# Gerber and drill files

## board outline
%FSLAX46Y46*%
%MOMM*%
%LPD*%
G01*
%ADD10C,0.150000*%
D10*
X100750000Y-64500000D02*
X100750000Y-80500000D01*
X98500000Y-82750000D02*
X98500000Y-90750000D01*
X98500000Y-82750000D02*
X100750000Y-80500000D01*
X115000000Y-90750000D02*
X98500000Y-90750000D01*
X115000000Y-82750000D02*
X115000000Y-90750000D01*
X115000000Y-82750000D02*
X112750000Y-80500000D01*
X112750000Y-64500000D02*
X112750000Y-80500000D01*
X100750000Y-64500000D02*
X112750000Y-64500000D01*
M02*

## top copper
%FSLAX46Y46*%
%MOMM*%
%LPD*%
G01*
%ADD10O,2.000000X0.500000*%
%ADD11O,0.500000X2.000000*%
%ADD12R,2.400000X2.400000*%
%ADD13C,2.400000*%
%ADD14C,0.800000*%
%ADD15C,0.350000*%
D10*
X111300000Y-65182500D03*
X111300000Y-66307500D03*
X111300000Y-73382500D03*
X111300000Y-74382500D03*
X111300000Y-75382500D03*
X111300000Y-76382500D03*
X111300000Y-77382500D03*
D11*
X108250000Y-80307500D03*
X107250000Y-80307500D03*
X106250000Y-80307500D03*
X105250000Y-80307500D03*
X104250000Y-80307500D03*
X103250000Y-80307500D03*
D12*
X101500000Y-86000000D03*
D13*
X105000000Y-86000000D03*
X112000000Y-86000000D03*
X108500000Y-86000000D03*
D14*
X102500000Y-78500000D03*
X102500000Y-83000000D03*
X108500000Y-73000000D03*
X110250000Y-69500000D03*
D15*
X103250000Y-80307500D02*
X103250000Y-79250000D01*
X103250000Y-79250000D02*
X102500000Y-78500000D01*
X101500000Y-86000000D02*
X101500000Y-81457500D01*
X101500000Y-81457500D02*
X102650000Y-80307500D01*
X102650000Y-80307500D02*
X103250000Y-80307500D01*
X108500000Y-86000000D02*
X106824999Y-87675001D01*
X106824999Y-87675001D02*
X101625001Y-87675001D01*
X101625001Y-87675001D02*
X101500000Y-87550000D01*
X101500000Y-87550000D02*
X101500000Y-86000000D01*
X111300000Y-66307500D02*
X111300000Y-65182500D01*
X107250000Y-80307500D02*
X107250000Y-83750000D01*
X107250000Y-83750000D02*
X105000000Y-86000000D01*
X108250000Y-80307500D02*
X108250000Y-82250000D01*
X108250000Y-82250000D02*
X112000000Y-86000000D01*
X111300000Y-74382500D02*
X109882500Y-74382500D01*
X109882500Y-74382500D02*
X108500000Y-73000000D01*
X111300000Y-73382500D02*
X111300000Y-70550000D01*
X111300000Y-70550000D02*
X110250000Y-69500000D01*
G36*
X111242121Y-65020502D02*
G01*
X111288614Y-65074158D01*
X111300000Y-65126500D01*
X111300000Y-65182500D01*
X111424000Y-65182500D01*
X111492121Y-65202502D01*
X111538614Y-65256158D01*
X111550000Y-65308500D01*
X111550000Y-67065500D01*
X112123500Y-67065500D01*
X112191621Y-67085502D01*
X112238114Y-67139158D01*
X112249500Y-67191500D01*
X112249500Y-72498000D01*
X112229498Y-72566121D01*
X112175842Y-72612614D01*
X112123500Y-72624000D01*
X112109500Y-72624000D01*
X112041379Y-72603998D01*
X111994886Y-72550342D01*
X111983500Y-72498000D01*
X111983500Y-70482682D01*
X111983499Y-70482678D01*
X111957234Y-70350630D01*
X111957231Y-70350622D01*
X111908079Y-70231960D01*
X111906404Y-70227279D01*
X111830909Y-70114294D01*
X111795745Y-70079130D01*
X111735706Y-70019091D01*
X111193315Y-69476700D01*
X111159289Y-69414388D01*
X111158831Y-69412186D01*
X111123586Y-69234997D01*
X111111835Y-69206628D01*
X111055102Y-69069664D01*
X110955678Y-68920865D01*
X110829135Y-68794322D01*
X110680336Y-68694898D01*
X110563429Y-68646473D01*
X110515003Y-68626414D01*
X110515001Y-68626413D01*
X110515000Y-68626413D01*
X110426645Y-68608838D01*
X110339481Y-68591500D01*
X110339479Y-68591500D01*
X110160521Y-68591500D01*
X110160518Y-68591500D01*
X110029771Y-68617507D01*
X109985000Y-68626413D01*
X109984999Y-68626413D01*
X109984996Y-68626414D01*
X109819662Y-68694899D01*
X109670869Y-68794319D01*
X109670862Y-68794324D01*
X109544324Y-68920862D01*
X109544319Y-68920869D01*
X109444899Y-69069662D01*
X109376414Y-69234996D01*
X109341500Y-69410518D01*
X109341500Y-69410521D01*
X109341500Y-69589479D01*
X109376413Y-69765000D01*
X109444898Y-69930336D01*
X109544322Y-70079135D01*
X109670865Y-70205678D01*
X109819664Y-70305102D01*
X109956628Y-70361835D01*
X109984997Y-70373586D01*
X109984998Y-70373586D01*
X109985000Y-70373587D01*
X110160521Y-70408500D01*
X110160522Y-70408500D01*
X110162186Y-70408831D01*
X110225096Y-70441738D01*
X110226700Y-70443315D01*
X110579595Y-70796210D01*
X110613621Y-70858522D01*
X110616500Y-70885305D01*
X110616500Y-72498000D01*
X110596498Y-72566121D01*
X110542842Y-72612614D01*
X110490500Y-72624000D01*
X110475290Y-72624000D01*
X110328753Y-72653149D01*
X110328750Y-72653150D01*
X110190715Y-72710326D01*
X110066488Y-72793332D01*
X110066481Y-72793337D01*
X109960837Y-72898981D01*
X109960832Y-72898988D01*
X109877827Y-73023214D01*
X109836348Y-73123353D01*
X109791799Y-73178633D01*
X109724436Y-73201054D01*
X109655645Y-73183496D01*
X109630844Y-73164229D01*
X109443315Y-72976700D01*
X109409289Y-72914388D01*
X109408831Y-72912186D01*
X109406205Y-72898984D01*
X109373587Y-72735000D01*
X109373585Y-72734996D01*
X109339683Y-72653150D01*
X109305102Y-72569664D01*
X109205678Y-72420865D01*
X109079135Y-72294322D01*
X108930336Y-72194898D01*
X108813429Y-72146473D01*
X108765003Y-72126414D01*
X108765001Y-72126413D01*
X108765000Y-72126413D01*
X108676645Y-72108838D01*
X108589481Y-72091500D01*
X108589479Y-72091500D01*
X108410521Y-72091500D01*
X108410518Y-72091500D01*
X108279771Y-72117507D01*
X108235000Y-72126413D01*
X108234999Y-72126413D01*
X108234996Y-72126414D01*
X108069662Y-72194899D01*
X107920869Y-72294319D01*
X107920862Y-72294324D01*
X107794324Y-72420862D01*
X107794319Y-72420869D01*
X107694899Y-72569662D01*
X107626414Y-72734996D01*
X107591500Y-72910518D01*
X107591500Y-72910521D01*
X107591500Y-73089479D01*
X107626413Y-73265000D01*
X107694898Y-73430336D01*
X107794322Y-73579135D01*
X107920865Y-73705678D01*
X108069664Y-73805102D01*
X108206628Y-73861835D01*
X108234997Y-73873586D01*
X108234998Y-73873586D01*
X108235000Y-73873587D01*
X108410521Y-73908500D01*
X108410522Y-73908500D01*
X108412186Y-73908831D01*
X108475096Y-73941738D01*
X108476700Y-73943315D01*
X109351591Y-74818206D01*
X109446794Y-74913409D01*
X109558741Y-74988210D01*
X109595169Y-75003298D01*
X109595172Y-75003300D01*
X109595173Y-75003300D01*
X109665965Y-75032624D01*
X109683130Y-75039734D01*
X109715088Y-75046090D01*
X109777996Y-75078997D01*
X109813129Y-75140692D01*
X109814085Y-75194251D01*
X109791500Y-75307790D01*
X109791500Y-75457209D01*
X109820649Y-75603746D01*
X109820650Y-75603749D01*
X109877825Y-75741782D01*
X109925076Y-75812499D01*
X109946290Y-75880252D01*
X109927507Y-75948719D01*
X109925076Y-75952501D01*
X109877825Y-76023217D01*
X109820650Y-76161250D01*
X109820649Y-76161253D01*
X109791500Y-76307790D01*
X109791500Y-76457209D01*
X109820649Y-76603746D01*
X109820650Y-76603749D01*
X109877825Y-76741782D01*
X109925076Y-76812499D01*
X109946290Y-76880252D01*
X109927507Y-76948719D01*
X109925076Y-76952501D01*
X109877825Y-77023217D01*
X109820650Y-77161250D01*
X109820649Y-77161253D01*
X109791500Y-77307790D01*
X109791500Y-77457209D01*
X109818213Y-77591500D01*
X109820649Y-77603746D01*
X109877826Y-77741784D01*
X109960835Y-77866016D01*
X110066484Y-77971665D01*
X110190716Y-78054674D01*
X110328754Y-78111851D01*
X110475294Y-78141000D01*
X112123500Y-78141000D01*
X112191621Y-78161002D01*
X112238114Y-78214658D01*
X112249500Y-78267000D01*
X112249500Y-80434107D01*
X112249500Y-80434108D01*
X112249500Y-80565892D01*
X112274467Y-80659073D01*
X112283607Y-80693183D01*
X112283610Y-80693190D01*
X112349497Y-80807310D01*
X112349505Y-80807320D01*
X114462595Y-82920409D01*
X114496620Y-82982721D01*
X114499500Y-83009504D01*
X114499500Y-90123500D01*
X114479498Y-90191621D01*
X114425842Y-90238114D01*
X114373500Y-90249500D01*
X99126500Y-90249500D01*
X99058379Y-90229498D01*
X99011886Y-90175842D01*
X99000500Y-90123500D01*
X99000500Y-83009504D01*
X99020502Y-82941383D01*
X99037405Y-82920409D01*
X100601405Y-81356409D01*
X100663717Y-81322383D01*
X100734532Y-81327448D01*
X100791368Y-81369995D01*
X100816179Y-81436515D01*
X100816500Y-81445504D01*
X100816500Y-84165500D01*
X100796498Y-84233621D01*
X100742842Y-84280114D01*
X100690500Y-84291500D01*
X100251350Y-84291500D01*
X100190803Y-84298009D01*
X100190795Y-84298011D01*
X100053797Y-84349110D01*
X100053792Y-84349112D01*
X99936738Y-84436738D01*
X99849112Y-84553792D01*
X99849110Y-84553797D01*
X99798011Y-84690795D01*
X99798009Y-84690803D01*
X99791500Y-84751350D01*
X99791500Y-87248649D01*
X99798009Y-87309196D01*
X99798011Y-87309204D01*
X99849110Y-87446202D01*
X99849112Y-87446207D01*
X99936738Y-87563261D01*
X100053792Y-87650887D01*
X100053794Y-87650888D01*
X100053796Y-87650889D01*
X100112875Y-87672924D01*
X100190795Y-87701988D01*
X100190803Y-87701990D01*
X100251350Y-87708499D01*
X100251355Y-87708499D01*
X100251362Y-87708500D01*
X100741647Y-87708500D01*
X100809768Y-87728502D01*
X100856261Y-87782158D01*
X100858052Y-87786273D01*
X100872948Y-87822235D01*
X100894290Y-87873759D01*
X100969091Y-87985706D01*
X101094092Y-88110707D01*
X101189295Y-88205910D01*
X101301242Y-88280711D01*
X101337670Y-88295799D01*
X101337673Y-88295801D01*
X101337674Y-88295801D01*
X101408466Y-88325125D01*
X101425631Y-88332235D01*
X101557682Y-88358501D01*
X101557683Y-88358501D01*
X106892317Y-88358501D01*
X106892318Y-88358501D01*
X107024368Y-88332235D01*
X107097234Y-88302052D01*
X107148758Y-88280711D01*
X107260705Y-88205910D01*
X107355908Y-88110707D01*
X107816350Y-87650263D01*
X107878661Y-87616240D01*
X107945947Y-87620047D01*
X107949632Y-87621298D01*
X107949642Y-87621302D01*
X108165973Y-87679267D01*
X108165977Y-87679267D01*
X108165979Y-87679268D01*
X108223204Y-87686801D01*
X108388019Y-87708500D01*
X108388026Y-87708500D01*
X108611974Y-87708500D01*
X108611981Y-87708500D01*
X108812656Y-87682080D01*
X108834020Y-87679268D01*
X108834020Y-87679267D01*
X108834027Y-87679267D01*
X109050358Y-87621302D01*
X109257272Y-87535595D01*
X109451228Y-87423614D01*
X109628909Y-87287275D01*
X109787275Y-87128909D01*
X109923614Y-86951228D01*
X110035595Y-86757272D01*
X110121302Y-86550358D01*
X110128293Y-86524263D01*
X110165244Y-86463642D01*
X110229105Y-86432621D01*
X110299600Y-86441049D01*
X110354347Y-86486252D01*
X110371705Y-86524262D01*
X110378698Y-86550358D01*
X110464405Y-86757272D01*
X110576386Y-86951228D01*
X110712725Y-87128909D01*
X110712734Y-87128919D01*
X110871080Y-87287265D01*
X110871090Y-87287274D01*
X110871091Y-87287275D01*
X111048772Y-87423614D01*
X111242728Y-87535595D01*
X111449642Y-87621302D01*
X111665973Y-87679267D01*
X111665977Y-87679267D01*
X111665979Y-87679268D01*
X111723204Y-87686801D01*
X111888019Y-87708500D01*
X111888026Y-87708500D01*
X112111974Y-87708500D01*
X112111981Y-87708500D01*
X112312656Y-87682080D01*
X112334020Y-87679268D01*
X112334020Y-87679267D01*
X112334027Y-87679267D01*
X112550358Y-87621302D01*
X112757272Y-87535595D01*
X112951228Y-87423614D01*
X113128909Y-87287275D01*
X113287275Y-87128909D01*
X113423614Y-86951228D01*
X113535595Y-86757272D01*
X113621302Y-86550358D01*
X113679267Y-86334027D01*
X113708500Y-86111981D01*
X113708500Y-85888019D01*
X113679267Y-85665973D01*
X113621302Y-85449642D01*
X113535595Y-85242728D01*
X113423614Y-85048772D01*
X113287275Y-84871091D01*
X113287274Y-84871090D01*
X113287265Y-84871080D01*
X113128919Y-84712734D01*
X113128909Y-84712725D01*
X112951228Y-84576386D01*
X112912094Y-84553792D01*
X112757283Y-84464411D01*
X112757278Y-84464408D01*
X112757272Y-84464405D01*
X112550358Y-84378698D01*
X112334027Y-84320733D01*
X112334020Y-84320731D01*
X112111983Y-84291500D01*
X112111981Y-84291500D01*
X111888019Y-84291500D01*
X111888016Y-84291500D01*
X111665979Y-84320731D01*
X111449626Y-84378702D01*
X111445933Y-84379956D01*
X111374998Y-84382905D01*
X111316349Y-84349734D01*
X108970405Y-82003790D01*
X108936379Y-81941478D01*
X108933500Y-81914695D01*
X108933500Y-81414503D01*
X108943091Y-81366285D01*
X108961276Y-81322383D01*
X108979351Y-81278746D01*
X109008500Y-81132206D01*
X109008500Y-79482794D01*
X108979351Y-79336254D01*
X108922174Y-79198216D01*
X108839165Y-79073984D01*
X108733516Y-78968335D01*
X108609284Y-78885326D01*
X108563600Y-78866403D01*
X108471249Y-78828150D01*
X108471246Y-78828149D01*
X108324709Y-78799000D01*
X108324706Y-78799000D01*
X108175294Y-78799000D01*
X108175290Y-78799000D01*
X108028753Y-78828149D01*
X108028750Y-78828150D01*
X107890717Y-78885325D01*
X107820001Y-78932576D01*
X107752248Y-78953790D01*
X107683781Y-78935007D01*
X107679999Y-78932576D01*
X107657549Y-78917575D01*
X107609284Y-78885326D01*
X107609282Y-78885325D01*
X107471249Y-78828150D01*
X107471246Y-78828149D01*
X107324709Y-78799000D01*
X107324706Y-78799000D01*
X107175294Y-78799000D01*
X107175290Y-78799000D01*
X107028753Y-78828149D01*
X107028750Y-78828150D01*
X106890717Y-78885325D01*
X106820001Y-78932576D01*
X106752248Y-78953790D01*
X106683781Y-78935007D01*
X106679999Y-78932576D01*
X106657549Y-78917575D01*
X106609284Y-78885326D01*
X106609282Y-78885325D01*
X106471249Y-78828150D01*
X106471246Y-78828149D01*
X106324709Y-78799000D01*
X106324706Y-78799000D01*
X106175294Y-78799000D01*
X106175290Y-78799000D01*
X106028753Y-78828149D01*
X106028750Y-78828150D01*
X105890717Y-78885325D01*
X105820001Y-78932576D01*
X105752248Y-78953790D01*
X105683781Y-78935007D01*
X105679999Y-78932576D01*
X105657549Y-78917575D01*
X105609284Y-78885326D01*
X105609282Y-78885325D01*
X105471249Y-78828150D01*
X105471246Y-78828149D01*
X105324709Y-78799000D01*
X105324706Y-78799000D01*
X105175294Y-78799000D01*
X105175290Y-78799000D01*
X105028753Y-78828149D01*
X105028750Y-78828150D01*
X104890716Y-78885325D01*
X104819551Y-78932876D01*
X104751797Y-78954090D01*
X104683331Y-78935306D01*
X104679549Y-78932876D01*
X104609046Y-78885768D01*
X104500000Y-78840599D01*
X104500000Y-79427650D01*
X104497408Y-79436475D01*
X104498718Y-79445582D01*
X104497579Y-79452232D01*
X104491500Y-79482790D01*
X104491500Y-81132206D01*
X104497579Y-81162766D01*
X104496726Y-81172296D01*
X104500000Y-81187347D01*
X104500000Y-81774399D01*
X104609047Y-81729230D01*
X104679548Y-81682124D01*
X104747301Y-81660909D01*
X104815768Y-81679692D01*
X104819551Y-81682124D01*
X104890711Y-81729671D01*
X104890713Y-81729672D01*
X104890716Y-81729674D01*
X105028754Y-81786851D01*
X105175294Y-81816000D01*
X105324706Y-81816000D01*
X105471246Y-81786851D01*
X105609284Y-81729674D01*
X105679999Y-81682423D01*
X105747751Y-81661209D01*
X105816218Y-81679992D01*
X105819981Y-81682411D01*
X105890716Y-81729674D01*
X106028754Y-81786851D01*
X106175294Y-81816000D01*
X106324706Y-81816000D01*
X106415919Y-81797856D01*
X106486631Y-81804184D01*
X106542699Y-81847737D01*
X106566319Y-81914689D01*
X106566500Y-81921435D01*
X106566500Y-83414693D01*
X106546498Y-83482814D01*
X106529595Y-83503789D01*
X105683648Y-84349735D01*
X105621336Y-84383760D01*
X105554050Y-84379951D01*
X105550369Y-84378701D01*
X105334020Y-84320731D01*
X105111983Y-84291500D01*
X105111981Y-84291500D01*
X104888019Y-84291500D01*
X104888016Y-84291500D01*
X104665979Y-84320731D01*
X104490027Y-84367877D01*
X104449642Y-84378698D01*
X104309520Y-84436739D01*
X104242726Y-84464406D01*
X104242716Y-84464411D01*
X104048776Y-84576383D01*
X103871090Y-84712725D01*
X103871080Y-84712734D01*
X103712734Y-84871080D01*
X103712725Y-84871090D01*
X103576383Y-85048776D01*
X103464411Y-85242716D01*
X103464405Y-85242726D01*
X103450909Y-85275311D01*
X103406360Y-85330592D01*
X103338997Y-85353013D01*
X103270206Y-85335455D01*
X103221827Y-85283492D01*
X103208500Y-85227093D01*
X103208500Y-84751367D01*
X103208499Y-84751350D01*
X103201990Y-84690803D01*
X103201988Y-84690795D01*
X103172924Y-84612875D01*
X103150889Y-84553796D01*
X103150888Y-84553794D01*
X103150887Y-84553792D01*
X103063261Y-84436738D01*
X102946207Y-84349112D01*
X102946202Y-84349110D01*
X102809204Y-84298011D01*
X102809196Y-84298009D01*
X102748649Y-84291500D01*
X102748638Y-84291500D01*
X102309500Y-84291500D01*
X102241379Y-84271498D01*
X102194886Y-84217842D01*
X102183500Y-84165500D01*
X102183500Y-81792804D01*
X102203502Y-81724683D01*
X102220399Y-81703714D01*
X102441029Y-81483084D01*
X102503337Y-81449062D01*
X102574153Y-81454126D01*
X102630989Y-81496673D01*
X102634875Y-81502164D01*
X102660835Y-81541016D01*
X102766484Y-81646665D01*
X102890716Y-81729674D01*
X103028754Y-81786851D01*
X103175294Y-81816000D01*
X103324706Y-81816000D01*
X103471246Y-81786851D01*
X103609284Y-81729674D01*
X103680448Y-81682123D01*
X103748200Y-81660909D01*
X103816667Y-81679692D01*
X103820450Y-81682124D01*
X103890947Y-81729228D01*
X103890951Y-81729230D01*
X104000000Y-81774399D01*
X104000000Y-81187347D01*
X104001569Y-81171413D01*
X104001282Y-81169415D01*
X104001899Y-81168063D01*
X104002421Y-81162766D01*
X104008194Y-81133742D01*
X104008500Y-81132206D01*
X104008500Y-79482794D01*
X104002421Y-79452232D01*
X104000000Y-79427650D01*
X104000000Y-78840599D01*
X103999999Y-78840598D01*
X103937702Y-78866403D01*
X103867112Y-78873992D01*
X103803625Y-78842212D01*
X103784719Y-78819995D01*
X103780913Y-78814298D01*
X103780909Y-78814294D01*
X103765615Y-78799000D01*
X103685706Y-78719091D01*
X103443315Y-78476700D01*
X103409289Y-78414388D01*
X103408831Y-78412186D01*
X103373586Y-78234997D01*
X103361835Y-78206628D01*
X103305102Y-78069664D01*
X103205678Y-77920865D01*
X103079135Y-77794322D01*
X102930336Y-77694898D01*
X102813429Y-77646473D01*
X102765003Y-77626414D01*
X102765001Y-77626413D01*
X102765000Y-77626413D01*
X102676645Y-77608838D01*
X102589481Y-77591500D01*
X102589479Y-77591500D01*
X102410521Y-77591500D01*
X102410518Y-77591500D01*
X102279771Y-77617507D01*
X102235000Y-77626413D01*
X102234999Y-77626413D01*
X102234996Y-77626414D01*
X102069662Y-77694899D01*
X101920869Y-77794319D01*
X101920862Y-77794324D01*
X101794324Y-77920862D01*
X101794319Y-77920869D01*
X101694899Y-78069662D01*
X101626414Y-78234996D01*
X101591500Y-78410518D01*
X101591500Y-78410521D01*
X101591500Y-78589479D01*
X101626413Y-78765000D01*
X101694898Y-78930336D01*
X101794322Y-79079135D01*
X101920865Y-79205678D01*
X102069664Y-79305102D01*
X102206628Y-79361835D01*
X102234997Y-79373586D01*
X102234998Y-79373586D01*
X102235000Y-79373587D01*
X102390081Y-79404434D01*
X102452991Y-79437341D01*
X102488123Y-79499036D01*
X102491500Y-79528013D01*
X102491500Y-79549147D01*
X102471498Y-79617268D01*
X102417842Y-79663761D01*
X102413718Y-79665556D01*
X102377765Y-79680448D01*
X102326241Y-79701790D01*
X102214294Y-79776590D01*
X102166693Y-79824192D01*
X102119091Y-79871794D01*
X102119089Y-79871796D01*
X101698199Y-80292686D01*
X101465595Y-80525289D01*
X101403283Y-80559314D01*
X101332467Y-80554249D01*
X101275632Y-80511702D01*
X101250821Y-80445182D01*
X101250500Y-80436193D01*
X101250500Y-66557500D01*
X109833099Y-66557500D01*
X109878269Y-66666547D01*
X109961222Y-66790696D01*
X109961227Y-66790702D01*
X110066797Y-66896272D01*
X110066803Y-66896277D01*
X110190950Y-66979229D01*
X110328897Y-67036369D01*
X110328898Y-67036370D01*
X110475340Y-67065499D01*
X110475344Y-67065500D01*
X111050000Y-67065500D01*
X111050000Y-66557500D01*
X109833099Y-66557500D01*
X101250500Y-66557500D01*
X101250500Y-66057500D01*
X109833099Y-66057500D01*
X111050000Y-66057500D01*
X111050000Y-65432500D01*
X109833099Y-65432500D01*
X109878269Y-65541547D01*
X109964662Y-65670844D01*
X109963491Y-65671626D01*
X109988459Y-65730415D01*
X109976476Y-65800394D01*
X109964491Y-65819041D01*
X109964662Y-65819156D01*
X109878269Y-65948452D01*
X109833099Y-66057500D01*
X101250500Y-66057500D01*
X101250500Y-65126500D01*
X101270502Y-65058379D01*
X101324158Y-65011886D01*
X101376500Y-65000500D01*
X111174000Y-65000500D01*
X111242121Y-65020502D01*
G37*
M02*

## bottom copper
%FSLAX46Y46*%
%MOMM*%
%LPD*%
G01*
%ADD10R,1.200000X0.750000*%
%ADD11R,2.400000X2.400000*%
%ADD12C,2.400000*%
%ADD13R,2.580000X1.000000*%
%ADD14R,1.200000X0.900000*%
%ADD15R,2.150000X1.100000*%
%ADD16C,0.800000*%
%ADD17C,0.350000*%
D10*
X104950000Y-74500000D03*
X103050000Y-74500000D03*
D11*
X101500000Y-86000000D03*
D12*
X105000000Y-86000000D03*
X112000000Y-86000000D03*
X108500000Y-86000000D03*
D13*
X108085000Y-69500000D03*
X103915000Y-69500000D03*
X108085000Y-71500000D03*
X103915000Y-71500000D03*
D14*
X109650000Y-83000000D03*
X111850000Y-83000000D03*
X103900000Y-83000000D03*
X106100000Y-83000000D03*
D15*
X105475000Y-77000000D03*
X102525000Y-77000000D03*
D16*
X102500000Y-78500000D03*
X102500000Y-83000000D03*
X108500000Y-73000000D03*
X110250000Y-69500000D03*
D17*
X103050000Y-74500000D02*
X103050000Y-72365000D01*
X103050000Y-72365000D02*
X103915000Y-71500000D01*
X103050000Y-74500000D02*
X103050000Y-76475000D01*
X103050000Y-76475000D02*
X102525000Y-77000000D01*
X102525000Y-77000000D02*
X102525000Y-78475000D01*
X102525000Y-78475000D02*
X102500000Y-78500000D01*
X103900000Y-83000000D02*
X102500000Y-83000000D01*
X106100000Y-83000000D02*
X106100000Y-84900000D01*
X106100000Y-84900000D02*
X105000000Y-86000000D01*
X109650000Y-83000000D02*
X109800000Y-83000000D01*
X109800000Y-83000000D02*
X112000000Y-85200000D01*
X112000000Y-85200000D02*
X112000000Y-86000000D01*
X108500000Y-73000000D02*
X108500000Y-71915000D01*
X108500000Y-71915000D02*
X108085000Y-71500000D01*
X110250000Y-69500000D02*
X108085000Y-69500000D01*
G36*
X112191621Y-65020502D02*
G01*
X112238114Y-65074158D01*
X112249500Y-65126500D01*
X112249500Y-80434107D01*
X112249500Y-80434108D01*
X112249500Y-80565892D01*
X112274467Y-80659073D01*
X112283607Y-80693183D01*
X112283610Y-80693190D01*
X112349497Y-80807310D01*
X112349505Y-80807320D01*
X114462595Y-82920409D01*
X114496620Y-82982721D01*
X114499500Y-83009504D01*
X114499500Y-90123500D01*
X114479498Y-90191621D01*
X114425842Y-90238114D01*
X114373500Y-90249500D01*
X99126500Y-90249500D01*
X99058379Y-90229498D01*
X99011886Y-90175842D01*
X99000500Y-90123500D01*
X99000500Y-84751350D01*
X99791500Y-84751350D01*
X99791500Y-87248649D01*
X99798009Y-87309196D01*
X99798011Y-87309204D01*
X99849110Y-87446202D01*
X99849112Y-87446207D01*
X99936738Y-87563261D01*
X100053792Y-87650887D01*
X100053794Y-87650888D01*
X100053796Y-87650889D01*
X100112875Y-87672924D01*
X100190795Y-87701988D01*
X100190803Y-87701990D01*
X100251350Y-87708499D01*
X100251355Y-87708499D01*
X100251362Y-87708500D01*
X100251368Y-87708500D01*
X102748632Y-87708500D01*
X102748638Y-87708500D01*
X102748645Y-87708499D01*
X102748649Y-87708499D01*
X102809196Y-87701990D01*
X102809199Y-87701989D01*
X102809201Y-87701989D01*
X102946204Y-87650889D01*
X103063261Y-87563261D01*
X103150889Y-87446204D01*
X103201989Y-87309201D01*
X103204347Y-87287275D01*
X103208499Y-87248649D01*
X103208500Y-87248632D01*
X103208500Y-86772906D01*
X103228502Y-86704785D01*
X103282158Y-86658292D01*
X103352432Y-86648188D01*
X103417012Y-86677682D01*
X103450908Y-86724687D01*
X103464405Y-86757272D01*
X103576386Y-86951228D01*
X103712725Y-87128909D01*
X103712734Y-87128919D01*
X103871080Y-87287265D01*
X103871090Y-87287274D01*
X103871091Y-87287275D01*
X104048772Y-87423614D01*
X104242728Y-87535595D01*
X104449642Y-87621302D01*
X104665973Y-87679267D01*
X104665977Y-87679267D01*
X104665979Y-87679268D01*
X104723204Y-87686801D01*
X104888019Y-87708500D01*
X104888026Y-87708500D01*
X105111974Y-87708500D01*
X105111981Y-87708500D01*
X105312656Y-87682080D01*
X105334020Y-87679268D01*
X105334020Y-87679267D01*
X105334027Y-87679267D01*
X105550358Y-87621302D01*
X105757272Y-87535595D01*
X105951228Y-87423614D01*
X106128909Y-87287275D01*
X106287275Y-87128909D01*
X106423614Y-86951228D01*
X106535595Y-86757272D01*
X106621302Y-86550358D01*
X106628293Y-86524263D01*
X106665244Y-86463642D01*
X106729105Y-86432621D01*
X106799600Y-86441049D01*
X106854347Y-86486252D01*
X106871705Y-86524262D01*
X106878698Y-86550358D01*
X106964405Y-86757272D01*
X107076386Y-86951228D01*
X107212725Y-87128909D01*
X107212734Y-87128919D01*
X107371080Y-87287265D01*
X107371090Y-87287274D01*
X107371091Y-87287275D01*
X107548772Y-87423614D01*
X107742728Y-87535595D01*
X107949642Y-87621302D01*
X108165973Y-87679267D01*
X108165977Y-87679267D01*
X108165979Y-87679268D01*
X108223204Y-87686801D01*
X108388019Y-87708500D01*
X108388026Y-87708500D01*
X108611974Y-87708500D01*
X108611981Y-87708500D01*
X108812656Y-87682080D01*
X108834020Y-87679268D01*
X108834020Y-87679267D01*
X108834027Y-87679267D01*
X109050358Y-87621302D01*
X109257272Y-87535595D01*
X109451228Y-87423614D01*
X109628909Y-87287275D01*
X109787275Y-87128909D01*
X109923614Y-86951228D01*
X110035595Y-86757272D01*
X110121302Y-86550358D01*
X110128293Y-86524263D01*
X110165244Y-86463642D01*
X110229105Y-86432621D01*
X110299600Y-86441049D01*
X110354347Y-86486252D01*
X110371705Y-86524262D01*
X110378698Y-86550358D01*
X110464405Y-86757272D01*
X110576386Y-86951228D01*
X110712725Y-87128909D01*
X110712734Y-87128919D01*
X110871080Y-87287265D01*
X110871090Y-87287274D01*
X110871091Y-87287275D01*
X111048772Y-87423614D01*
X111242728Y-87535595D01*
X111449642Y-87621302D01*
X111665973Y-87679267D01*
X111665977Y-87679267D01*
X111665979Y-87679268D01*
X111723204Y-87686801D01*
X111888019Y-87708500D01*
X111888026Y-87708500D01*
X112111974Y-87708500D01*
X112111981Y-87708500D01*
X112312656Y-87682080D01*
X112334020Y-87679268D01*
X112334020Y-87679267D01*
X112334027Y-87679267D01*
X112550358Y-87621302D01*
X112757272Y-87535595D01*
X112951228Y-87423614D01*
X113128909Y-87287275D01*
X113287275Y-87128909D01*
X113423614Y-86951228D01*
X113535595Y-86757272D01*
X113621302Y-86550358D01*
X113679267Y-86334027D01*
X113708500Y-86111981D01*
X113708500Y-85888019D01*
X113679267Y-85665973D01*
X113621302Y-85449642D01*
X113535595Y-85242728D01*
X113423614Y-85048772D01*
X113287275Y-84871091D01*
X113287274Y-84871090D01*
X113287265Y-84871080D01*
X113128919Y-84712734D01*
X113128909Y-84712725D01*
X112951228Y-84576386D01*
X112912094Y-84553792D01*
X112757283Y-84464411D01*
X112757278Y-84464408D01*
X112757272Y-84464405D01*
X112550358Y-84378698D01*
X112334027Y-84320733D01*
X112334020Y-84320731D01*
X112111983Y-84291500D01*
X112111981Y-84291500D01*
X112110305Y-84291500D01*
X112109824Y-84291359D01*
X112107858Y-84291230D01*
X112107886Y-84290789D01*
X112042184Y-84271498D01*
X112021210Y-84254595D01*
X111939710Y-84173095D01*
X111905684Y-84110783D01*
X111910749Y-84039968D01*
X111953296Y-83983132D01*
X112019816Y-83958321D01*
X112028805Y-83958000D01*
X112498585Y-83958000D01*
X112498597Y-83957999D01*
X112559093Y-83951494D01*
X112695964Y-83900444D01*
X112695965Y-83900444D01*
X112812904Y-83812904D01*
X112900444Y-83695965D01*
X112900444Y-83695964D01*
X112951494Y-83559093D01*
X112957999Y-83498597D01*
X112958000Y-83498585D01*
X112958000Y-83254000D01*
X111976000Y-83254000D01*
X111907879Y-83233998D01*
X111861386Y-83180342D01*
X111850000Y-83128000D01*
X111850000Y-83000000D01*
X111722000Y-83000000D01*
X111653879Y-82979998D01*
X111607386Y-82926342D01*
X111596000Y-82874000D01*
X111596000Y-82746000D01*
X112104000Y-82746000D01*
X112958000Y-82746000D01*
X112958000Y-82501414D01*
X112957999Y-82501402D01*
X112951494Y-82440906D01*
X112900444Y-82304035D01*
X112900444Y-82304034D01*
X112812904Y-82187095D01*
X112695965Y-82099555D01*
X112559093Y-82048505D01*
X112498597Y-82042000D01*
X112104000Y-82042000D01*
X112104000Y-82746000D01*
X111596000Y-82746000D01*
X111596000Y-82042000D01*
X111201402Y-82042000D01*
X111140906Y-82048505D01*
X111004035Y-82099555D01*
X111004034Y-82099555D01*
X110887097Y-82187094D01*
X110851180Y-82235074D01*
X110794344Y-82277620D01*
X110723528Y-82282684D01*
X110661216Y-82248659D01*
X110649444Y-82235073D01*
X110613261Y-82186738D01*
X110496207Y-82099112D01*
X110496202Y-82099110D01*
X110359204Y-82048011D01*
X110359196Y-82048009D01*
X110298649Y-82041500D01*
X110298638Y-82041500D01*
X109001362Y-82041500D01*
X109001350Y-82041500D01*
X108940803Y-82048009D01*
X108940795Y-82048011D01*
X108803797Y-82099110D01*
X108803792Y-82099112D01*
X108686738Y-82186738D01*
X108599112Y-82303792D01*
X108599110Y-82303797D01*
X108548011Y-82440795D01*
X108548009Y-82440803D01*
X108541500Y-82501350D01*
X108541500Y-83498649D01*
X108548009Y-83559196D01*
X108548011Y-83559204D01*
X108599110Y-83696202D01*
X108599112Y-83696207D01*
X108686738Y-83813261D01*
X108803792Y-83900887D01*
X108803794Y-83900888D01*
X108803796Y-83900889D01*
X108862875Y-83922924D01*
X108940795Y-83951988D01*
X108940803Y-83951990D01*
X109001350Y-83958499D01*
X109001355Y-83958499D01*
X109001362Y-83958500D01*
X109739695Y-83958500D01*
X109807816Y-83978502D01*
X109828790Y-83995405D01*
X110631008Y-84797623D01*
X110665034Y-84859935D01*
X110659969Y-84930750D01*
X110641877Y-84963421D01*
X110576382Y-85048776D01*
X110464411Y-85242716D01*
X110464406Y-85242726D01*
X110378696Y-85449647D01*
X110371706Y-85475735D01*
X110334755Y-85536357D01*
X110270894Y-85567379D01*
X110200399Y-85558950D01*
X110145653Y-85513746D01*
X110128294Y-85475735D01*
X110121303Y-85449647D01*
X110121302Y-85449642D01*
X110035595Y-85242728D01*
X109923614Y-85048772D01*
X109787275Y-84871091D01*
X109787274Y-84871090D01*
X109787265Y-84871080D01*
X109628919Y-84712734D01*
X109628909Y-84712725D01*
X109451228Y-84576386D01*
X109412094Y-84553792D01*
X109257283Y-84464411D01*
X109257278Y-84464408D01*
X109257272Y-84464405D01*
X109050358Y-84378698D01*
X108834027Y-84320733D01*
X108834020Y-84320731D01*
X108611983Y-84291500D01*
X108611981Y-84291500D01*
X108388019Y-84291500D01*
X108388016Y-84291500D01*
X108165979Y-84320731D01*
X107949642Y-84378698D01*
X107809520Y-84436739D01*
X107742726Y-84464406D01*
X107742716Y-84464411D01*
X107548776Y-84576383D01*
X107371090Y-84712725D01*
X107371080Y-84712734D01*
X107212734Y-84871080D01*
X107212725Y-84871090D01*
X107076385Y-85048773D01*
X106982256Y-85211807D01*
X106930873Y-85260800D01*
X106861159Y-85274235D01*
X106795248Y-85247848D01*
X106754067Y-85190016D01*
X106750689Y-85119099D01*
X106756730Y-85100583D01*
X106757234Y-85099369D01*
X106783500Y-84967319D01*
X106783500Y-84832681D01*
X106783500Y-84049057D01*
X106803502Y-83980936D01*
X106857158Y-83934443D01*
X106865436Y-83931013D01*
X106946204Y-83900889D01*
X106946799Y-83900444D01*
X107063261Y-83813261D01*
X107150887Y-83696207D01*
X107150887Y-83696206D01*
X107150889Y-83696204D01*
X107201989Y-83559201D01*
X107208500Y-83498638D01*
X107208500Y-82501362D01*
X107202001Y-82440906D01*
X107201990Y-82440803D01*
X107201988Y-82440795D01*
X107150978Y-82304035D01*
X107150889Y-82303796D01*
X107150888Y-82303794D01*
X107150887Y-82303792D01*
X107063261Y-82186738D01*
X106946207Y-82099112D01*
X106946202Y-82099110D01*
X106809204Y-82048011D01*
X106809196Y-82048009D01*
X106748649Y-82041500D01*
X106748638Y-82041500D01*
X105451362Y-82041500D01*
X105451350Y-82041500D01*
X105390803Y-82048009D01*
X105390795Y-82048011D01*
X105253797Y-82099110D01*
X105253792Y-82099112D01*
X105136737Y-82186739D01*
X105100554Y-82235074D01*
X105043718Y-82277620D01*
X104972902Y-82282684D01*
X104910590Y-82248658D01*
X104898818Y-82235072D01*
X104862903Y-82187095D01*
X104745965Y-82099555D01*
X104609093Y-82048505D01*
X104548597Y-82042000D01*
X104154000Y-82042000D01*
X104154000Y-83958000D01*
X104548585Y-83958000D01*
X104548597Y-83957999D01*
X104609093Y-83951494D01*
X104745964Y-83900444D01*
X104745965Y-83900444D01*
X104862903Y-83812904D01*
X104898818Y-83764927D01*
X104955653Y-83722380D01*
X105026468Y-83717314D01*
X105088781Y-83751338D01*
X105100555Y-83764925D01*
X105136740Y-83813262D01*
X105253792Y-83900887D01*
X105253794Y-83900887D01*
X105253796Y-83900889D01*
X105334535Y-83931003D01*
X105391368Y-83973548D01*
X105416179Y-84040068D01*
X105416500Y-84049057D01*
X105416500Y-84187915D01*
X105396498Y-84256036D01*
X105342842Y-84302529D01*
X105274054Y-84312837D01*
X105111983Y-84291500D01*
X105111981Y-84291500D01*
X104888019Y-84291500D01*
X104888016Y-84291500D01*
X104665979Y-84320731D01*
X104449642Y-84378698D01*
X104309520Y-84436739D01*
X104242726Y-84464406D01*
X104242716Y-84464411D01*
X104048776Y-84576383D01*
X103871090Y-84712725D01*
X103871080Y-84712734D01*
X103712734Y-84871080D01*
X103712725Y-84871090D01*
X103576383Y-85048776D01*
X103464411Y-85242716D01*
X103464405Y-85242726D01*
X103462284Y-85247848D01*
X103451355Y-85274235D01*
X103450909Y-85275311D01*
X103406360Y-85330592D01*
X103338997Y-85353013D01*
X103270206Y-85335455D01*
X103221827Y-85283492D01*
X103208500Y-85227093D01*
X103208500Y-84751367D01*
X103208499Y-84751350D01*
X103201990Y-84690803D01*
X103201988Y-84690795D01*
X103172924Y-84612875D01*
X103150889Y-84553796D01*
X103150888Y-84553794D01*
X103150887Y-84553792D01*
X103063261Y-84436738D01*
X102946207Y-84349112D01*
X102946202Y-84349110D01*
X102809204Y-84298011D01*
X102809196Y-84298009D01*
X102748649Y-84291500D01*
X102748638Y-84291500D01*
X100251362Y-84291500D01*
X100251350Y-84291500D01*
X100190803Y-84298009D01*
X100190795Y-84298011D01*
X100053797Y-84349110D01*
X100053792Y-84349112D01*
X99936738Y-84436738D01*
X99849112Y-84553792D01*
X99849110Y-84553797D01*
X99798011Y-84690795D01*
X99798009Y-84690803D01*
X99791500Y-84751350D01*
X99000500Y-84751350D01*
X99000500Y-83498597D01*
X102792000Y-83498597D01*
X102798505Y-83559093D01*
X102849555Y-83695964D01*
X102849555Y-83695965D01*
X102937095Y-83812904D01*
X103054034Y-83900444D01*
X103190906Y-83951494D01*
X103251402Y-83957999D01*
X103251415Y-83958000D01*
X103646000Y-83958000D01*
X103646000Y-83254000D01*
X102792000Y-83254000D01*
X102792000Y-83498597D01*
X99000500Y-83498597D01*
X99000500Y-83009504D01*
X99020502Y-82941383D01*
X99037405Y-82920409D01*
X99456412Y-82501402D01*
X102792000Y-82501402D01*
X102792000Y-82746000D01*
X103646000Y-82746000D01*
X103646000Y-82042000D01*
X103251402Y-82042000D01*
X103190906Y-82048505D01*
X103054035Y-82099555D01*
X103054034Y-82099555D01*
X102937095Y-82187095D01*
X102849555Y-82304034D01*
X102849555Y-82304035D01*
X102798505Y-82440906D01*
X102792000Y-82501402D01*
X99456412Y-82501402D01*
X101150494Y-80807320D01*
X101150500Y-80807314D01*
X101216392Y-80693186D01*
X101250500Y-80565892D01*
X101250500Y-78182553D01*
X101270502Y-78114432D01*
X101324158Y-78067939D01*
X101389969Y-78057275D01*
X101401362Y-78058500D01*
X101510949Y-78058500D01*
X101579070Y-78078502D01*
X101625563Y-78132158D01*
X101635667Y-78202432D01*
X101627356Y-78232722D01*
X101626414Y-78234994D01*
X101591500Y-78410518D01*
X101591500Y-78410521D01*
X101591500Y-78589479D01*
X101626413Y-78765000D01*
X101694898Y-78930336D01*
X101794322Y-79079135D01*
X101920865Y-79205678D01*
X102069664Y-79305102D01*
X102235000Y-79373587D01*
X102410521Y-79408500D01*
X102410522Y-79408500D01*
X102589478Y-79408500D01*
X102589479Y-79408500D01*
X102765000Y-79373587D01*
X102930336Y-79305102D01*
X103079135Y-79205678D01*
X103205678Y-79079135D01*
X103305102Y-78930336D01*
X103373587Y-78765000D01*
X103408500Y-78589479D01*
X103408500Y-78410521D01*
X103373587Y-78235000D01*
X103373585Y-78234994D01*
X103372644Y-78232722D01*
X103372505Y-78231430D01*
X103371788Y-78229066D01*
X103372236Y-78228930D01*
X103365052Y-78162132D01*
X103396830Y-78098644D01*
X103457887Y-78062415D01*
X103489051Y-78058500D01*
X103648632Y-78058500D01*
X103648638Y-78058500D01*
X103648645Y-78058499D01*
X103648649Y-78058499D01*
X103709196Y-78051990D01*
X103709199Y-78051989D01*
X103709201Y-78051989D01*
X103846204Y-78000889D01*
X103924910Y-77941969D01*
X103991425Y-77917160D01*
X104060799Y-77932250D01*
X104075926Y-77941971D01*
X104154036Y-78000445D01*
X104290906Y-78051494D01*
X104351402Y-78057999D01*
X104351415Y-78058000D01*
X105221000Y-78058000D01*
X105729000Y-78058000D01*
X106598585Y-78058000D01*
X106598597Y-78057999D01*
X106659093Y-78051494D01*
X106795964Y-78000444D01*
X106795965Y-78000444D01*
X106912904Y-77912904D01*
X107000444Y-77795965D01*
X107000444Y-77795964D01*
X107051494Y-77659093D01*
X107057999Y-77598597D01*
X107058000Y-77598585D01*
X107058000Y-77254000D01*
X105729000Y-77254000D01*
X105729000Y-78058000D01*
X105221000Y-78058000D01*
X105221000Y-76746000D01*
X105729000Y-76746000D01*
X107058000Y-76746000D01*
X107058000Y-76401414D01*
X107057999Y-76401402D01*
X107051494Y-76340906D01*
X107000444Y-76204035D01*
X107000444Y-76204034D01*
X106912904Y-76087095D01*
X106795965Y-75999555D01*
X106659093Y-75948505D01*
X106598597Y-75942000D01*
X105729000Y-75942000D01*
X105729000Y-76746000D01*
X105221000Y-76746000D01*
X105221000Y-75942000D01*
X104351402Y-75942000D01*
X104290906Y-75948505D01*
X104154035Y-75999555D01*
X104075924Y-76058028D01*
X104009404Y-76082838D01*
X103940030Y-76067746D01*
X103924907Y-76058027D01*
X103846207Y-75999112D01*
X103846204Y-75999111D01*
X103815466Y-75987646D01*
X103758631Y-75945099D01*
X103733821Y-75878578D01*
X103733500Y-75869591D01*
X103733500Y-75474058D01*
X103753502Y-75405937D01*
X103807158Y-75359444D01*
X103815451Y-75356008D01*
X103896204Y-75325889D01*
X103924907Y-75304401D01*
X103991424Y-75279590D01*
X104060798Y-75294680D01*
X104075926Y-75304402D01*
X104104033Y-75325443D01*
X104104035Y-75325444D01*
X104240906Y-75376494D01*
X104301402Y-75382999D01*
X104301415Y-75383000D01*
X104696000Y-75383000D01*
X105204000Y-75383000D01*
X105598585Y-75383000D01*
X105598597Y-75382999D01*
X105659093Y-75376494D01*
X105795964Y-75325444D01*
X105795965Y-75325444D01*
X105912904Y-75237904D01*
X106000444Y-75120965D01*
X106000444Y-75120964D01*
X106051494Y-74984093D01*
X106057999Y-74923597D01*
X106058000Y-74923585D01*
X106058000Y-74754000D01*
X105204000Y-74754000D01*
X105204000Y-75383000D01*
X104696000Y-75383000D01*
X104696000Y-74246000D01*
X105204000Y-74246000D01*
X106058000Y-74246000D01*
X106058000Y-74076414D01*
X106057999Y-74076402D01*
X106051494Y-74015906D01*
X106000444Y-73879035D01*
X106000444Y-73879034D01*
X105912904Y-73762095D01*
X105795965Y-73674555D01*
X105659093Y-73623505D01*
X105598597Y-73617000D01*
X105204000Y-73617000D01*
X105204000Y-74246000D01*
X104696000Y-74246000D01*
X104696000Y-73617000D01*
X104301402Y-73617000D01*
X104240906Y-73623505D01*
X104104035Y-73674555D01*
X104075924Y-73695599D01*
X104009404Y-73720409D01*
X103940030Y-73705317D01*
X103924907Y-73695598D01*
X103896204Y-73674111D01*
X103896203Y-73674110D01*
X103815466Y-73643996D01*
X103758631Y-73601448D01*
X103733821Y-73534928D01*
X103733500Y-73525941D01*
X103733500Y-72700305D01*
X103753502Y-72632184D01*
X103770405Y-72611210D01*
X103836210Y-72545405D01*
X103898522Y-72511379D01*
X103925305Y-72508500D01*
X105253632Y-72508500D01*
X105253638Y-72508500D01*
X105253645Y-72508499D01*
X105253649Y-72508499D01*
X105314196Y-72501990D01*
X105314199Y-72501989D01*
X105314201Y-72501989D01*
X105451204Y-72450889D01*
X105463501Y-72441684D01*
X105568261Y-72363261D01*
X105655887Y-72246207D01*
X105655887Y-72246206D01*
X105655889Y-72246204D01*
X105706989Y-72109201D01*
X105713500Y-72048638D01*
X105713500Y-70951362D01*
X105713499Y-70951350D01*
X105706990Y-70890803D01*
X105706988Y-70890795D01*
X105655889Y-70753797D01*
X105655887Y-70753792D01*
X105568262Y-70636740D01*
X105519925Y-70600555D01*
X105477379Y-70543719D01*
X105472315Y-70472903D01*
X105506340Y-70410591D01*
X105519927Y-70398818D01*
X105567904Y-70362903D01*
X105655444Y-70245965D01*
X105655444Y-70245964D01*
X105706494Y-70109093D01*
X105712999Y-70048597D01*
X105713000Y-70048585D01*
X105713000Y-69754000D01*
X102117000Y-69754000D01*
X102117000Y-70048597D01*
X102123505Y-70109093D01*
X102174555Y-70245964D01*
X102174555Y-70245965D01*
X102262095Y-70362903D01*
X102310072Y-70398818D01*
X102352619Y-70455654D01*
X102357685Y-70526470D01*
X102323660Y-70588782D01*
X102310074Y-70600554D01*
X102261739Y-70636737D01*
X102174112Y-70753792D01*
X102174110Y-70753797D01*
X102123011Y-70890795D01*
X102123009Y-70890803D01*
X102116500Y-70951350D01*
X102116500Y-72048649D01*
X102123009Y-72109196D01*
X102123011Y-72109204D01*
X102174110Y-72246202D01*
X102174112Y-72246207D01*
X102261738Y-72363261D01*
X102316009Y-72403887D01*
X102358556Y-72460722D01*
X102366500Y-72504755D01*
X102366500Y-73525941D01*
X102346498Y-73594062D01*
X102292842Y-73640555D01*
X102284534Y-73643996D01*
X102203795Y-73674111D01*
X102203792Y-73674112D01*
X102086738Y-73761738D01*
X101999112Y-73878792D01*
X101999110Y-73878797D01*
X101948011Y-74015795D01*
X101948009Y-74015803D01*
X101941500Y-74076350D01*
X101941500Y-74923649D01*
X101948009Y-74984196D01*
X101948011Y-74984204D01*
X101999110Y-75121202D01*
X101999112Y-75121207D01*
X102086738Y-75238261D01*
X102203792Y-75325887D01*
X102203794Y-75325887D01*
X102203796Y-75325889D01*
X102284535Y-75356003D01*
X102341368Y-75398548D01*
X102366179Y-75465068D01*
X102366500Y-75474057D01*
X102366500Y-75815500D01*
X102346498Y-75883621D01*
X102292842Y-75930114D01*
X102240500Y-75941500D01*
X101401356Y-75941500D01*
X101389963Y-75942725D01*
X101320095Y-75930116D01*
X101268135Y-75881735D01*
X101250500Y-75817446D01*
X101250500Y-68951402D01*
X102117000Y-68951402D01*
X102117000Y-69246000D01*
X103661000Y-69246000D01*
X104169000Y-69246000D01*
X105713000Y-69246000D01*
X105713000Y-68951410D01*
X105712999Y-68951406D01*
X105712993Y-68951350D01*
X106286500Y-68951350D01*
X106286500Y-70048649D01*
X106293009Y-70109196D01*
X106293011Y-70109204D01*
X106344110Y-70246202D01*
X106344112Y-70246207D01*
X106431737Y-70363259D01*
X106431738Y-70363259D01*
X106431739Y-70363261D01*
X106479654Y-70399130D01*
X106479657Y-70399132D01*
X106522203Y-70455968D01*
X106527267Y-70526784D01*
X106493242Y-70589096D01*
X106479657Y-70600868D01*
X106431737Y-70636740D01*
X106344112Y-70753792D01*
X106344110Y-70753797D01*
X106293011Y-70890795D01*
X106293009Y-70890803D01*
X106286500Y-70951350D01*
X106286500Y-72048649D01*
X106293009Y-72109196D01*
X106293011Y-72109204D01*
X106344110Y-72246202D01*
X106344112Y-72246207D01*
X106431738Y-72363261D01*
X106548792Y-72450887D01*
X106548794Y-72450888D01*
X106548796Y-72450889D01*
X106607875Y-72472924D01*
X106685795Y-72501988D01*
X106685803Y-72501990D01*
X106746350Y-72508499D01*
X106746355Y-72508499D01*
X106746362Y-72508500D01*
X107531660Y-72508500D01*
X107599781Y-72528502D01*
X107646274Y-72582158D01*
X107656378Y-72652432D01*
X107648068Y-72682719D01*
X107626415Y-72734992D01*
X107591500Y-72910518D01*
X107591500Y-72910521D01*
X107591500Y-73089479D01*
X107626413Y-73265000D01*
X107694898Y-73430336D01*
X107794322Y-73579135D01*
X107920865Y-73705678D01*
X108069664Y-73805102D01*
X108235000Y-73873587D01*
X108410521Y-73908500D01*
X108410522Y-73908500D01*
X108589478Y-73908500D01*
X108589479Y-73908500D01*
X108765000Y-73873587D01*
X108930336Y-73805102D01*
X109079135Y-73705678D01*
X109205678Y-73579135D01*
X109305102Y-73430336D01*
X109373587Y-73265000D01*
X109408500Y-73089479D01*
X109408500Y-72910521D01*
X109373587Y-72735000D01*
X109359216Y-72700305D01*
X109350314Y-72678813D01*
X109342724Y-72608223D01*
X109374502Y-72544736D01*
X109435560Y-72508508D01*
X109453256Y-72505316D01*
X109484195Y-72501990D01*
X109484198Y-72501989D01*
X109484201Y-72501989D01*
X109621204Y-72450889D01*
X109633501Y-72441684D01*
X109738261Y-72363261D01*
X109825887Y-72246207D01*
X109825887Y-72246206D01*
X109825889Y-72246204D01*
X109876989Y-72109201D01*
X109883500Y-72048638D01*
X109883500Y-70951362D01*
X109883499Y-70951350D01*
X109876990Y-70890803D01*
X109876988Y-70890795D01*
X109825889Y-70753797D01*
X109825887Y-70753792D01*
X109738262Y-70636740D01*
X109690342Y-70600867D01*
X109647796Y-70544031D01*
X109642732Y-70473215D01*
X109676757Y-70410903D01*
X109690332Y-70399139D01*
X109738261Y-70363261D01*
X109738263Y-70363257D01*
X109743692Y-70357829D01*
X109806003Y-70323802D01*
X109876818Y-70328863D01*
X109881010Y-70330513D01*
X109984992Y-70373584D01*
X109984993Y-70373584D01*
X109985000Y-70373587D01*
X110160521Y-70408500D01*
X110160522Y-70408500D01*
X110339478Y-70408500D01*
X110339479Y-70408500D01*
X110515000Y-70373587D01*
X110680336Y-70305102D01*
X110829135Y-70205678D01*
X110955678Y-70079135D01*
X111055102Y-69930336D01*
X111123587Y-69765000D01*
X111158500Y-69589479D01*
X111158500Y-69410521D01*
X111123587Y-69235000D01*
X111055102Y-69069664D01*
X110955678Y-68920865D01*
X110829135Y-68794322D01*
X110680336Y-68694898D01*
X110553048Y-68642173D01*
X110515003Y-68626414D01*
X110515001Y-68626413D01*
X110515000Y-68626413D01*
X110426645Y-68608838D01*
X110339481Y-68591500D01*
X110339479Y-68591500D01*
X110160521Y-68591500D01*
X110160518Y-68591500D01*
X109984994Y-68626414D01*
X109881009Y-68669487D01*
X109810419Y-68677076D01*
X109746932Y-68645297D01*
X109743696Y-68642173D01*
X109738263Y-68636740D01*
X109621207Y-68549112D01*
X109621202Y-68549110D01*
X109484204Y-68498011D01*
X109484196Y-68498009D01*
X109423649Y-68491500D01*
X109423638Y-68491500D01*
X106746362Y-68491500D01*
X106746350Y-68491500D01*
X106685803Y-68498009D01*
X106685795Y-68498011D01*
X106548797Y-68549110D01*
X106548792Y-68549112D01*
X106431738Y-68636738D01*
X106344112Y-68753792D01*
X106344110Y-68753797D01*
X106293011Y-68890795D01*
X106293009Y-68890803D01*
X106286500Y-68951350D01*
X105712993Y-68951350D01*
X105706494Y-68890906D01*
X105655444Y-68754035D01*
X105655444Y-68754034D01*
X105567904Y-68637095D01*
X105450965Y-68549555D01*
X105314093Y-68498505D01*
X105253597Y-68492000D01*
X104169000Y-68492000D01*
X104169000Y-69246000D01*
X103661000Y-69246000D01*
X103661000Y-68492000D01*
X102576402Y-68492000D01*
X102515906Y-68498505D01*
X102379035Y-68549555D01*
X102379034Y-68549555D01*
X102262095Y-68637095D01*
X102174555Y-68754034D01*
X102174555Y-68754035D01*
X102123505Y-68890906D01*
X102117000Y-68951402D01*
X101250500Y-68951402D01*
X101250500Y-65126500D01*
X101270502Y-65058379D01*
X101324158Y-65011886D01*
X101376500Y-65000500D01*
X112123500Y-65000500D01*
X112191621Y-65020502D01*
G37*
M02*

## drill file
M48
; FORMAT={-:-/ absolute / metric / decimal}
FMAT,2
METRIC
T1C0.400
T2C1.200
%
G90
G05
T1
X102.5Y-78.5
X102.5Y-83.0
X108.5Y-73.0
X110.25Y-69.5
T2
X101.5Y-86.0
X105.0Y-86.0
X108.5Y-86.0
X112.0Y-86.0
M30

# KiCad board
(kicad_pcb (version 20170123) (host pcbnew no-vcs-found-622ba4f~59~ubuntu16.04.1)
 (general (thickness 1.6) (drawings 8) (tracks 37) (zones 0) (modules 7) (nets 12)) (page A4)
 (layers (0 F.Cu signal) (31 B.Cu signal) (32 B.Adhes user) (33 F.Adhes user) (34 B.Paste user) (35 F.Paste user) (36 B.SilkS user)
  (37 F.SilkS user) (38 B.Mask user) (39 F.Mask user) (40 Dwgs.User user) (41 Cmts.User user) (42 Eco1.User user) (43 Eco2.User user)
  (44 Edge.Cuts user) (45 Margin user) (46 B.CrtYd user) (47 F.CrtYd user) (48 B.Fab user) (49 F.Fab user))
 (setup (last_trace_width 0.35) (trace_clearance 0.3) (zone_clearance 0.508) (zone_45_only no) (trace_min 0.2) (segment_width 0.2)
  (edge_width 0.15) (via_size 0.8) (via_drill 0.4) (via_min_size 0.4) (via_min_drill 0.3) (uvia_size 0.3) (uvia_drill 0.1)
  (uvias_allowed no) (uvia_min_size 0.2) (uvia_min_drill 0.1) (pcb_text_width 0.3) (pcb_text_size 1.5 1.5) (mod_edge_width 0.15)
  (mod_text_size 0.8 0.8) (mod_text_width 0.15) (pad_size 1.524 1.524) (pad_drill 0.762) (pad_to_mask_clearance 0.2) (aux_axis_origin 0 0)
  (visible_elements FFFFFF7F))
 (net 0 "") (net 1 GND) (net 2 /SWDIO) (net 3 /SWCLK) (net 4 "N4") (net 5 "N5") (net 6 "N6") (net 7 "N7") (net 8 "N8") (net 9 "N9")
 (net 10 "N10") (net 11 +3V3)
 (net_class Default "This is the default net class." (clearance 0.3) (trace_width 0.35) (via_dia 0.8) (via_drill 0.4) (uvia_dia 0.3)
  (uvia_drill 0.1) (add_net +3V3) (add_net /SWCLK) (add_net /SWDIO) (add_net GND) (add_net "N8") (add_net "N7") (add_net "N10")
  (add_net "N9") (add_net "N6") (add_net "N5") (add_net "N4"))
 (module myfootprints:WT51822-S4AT (layer F.Cu) (at 106.75 71.0575)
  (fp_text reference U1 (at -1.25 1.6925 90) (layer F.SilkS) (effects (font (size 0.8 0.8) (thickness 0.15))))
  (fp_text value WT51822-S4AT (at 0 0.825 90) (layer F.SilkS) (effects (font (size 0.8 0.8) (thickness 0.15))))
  (pad 13 smd oval (at 4.55 -5.875 90) (size 0.5 2) (layers F.Cu F.Paste F.Mask) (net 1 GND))
  (pad 12 smd oval (at 4.55 -4.75 90) (size 0.5 2) (layers F.Cu F.Paste F.Mask) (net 1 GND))
  (pad 11 smd oval (at 4.55 2.325 90) (size 0.5 2) (layers F.Cu F.Paste F.Mask) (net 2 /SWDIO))
  (pad 10 smd oval (at 4.55 3.325 90) (size 0.5 2) (layers F.Cu F.Paste F.Mask) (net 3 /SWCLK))
  (pad 9 smd oval (at 4.55 4.325 90) (size 0.5 2) (layers F.Cu F.Paste F.Mask) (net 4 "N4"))
  (pad 8 smd oval (at 4.55 5.325 90) (size 0.5 2) (layers F.Cu F.Paste F.Mask) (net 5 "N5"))
  (pad 7 smd oval (at 4.55 6.325 90) (size 0.5 2) (layers F.Cu F.Paste F.Mask) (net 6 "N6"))
  (pad 6 smd oval (at 1.5 9.25) (size 0.5 2) (layers F.Cu F.Paste F.Mask) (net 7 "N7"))
  (pad 5 smd oval (at 0.5 9.25) (size 0.5 2) (layers F.Cu F.Paste F.Mask) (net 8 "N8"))
  (pad 4 smd oval (at -0.5 9.25) (size 0.5 2) (layers F.Cu F.Paste F.Mask) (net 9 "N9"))
  (pad 3 smd oval (at -1.5 9.25) (size 0.5 2) (layers F.Cu F.Paste F.Mask) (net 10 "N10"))
  (pad 2 smd oval (at -2.5 9.25) (size 0.5 2) (layers F.Cu F.Paste F.Mask) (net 1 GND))
  (pad 1 smd oval (at -3.5 9.25) (size 0.5 2) (layers F.Cu F.Paste F.Mask) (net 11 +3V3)))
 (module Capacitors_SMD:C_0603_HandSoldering (layer B.Cu) (at 104 74.5)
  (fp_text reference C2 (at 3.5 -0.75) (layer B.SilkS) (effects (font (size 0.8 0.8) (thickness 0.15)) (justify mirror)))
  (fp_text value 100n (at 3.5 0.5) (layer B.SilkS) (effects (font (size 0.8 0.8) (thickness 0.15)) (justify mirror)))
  (pad 2 smd rect (at 0.95 0) (size 1.2 0.75) (layers B.Cu B.Paste B.Mask) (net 1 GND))
  (pad 1 smd rect (at -0.95 0) (size 1.2 0.75) (layers B.Cu B.Paste B.Mask) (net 11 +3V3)))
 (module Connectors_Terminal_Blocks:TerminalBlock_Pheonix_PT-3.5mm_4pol (layer F.Cu) (at 101.5 86)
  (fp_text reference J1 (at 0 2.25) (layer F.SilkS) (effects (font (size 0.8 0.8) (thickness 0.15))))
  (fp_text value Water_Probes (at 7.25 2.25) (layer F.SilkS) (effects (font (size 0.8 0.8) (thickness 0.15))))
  (pad 1 thru_hole rect (at 0 0) (size 2.4 2.4) (drill 1.2) (layers *.Cu *.Mask) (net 11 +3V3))
  (pad 2 thru_hole circle (at 3.5 0) (size 2.4 2.4) (drill 1.2) (layers *.Cu *.Mask) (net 8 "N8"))
  (pad 4 thru_hole circle (at 10.5 0) (size 2.4 2.4) (drill 1.2) (layers *.Cu *.Mask) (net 7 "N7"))
  (pad 3 thru_hole circle (at 7 0) (size 2.4 2.4) (drill 1.2) (layers *.Cu *.Mask) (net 11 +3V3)))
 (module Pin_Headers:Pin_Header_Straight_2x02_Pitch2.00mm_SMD (layer B.Cu) (at 106 70.5)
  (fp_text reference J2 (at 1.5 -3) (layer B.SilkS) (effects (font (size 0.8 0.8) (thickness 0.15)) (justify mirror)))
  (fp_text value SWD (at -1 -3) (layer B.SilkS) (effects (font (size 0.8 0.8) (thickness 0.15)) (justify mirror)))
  (pad 4 smd rect (at 2.085 -1) (size 2.58 1) (layers B.Cu B.Paste B.Mask) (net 2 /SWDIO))
  (pad 3 smd rect (at -2.085 -1) (size 2.58 1) (layers B.Cu B.Paste B.Mask) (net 1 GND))
  (pad 2 smd rect (at 2.085 1) (size 2.58 1) (layers B.Cu B.Paste B.Mask) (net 3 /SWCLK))
  (pad 1 smd rect (at -2.085 1) (size 2.58 1) (layers B.Cu B.Paste B.Mask) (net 11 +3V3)))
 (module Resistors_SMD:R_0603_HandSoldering (layer B.Cu) (at 110.75 83)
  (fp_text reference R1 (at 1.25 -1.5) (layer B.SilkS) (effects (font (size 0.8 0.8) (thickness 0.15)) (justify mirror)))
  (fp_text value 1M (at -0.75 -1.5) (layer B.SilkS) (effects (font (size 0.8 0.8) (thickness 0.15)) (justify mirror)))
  (pad 1 smd rect (at -1.1 0) (size 1.2 0.9) (layers B.Cu B.Paste B.Mask) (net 7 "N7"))
  (pad 2 smd rect (at 1.1 0) (size 1.2 0.9) (layers B.Cu B.Paste B.Mask) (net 1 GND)))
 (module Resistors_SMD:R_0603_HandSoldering (layer B.Cu) (at 105 83 180)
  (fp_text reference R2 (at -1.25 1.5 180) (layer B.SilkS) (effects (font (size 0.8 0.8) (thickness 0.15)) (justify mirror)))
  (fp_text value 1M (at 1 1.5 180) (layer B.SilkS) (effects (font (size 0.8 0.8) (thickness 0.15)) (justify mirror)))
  (pad 2 smd rect (at 1.1 0 180) (size 1.2 0.9) (layers B.Cu B.Paste B.Mask) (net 1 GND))
  (pad 1 smd rect (at -1.1 0 180) (size 1.2 0.9) (layers B.Cu B.Paste B.Mask) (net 8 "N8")))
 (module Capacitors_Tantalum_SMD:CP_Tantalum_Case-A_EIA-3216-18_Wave (layer B.Cu) (at 104 77)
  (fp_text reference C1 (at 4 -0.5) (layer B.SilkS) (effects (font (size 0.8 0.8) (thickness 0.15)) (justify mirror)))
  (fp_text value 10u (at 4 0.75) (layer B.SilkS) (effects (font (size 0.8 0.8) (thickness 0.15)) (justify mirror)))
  (pad 2 smd rect (at 1.475 0) (size 2.15 1.1) (layers B.Cu B.Paste B.Mask) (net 1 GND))
  (pad 1 smd rect (at -1.475 0) (size 2.15 1.1) (layers B.Cu B.Paste B.Mask) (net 11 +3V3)))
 (gr_line (start 100.75 64.5) (end 100.75 80.5) (layer Edge.Cuts) (width 0.15))
 (gr_line (start 98.5 82.75) (end 98.5 90.75) (layer Edge.Cuts) (width 0.15))
 (gr_line (start 98.5 82.75) (end 100.75 80.5) (layer Edge.Cuts) (width 0.15))
 (gr_line (start 115 90.75) (end 98.5 90.75) (layer Edge.Cuts) (width 0.15))
 (gr_line (start 115 82.75) (end 115 90.75) (layer Edge.Cuts) (width 0.15))
 (gr_line (start 115 82.75) (end 112.75 80.5) (layer Edge.Cuts) (width 0.15))
 (gr_line (start 112.75 64.5) (end 112.75 80.5) (layer Edge.Cuts) (width 0.15))
 (gr_line (start 100.75 64.5) (end 112.75 64.5) (layer Edge.Cuts) (width 0.15))
 (segment (start 103.05 74.5) (end 103.05 72.365) (width 0.35) (layer B.Cu) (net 11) (status 10))
 (segment (start 103.05 72.365) (end 103.915 71.5) (width 0.35) (layer B.Cu) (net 11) (status 20))
 (segment (start 103.05 74.5) (end 103.05 76.475) (width 0.35) (layer B.Cu) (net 11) (status 30))
 (segment (start 103.05 76.475) (end 102.525 77) (width 0.35) (layer B.Cu) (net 11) (status 30))
 (segment (start 103.25 80.3075) (end 103.25 79.25) (width 0.35) (layer F.Cu) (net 11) (status 10))
 (segment (start 103.25 79.25) (end 102.5 78.5) (width 0.35) (layer F.Cu) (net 11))
 (segment (start 102.525 77) (end 102.525 78.475) (width 0.35) (layer B.Cu) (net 11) (status 10))
 (segment (start 102.525 78.475) (end 102.5 78.5) (width 0.35) (layer B.Cu) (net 11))
 (via (at 102.5 78.5) (size 0.8) (drill 0.4) (layers F.Cu B.Cu) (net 11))
 (segment (start 101.5 86) (end 101.5 81.4575) (width 0.35) (layer F.Cu) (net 11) (status 10))
 (segment (start 101.5 81.4575) (end 102.65 80.3075) (width 0.35) (layer F.Cu) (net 11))
 (segment (start 102.65 80.3075) (end 103.25 80.3075) (width 0.35) (layer F.Cu) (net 11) (status 20))
 (segment (start 108.5 86) (end 106.824999 87.675001) (width 0.35) (layer F.Cu) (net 11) (status 10))
 (segment (start 106.824999 87.675001) (end 101.625001 87.675001) (width 0.35) (layer F.Cu) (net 11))
 (segment (start 101.625001 87.675001) (end 101.5 87.55) (width 0.35) (layer F.Cu) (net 11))
 (segment (start 101.5 87.55) (end 101.5 86) (width 0.35) (layer F.Cu) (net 11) (status 20))
 (segment (start 103.9 83) (end 102.5 83) (width 0.35) (layer B.Cu) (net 1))
 (via (at 102.5 83) (size 0.8) (drill 0.4) (layers F.Cu B.Cu) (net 1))
 (segment (start 111.3 66.3075) (end 111.3 65.1825) (width 0.35) (layer F.Cu) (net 1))
 (segment (start 106.1 83) (end 106.1 84.9) (width 0.35) (layer B.Cu) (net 8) (status 10))
 (segment (start 106.1 84.9) (end 105 86) (width 0.35) (layer B.Cu) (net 8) (status 20))
 (segment (start 107.25 80.3075) (end 107.25 83.75) (width 0.35) (layer F.Cu) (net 8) (status 10))
 (segment (start 107.25 83.75) (end 105 86) (width 0.35) (layer F.Cu) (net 8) (status 20))
 (segment (start 108.25 80.3075) (end 108.25 82.25) (width 0.35) (layer F.Cu) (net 7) (status 10))
 (segment (start 108.25 82.25) (end 112 86) (width 0.35) (layer F.Cu) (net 7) (status 20))
 (segment (start 109.65 83) (end 109.8 83) (width 0.35) (layer B.Cu) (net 7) (status 30))
 (segment (start 109.8 83) (end 112 85.2) (width 0.35) (layer B.Cu) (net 7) (status 30))
 (segment (start 112 85.2) (end 112 86) (width 0.35) (layer B.Cu) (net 7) (status 30))
 (segment (start 108.5 73) (end 108.5 71.915) (width 0.35) (layer B.Cu) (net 3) (status 20))
 (segment (start 108.5 71.915) (end 108.085 71.5) (width 0.35) (layer B.Cu) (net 3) (status 30))
 (segment (start 111.3 74.3825) (end 109.8825 74.3825) (width 0.35) (layer F.Cu) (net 3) (status 10))
 (segment (start 109.8825 74.3825) (end 108.5 73) (width 0.35) (layer F.Cu) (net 3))
 (via (at 108.5 73) (size 0.8) (drill 0.4) (layers F.Cu B.Cu) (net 3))
 (segment (start 110.25 69.5) (end 108.085 69.5) (width 0.35) (layer B.Cu) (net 2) (status 20))
 (segment (start 111.3 73.3825) (end 111.3 70.55) (width 0.35) (layer F.Cu) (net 2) (status 10))
 (segment (start 111.3 70.55) (end 110.25 69.5) (width 0.35) (layer F.Cu) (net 2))
 (via (at 110.25 69.5) (size 0.8) (drill 0.4) (layers F.Cu B.Cu) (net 2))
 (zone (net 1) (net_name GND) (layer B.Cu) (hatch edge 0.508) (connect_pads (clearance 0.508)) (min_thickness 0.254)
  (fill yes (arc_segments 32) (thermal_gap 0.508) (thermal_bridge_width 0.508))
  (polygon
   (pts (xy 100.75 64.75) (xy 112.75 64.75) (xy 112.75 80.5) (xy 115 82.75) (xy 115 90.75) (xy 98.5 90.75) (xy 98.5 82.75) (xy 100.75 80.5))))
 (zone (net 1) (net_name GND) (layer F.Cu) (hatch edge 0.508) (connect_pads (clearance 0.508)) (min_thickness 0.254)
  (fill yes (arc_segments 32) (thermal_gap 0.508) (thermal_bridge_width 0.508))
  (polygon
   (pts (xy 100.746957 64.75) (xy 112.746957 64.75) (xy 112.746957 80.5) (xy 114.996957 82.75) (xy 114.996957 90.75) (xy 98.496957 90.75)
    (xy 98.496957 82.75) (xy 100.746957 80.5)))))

